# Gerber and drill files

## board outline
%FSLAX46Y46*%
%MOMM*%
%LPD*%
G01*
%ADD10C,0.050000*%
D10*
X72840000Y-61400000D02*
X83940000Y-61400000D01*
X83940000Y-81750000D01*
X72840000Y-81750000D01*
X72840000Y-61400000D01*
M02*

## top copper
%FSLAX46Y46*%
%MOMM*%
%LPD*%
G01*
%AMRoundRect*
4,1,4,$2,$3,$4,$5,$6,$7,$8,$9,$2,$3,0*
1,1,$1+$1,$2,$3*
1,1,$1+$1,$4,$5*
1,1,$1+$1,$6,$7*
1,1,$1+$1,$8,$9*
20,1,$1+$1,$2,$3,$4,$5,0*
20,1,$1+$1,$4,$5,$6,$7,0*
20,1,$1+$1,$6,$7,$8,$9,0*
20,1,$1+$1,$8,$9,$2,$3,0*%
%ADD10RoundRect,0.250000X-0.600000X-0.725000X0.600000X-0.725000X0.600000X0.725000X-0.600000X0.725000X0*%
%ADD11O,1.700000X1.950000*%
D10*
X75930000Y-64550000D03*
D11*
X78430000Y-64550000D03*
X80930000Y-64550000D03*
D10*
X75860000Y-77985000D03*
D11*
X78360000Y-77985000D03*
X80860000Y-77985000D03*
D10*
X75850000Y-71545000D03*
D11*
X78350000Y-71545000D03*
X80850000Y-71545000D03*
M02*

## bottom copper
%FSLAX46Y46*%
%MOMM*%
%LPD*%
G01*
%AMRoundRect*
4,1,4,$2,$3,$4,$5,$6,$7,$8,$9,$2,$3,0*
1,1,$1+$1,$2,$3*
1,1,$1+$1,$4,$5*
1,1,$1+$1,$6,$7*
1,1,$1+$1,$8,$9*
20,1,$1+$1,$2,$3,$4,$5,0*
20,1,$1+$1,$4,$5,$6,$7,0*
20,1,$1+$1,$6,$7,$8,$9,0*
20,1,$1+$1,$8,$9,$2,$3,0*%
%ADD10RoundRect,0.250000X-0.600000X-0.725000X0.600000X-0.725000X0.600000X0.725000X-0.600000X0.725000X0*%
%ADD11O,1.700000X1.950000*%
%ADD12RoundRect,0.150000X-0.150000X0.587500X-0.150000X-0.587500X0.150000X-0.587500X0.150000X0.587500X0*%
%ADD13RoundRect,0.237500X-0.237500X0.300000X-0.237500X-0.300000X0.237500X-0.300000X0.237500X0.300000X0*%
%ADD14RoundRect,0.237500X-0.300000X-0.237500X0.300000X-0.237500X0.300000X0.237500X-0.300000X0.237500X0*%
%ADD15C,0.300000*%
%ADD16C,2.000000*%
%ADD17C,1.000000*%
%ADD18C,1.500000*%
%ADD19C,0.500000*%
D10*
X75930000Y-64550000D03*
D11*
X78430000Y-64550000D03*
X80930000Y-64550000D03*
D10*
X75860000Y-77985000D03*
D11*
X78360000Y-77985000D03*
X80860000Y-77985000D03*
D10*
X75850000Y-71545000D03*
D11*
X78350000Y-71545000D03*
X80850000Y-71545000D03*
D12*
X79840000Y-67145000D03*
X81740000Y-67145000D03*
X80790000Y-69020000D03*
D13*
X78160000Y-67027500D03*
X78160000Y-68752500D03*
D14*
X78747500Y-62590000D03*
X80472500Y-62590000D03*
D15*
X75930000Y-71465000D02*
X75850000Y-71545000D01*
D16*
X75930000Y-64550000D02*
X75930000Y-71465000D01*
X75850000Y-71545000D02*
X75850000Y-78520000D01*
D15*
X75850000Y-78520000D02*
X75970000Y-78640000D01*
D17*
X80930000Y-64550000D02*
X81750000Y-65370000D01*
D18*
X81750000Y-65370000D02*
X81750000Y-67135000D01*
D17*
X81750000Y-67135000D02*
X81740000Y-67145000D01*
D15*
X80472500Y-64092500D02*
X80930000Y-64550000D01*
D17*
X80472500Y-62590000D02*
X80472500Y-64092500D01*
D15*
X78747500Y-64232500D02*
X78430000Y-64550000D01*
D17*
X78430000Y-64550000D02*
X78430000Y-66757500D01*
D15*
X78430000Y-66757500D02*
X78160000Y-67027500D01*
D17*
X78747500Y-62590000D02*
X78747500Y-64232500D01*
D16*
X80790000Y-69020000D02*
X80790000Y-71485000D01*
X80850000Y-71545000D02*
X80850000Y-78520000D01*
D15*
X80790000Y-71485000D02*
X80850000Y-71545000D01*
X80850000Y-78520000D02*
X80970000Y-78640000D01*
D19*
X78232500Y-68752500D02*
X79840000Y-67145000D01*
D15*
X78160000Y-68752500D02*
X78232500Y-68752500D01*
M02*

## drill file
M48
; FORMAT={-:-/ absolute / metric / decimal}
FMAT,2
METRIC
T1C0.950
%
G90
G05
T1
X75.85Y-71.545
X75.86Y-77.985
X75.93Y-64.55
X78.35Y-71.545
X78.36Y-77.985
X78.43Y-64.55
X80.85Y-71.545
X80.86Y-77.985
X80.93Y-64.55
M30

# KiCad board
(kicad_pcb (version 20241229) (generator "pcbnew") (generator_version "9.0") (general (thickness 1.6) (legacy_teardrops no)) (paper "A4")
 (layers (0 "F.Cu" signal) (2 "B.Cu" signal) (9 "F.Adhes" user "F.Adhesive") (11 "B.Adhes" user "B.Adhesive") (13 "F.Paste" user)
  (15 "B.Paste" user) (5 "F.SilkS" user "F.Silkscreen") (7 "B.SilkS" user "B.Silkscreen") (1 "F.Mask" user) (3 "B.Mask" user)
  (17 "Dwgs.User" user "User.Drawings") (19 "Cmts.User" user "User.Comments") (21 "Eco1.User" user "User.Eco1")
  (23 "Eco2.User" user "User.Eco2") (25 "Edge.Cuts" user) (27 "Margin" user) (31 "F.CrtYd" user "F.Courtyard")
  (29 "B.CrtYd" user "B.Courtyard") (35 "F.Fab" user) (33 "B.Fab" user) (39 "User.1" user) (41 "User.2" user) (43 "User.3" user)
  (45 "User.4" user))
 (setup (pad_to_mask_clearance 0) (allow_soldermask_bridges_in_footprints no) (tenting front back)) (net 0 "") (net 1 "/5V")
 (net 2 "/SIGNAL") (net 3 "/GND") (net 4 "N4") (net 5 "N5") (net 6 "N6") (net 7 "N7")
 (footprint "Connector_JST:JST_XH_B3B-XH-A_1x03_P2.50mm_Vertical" (layer "F.Cu") (at 75.93 64.55)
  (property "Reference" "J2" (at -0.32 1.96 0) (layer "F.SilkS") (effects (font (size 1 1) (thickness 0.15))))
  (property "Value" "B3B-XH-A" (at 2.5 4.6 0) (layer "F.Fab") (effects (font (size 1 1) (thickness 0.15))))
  (pad "1" thru_hole roundrect (at 0 0) (size 1.7 1.95) (drill 0.95) (layers "*.Cu" "*.Mask") (remove_unused_layers no)
   (roundrect_rratio 0.147059) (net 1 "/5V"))
  (pad "2" thru_hole oval (at 2.5 0) (size 1.7 1.95) (drill 0.95) (layers "*.Cu" "*.Mask") (remove_unused_layers no) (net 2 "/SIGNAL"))
  (pad "3" thru_hole oval (at 5 0) (size 1.7 1.95) (drill 0.95) (layers "*.Cu" "*.Mask") (remove_unused_layers no) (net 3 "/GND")))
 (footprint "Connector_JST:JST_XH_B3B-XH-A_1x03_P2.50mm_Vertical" (layer "F.Cu") (at 75.86 77.985)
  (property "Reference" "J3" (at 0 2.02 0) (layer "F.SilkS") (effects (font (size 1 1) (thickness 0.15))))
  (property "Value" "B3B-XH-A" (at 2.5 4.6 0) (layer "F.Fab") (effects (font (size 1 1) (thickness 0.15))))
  (pad "1" thru_hole roundrect (at 0 0) (size 1.7 1.95) (drill 0.95) (layers "*.Cu" "*.Mask") (remove_unused_layers no)
   (roundrect_rratio 0.147059) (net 1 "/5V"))
  (pad "2" thru_hole oval (at 2.5 0) (size 1.7 1.95) (drill 0.95) (layers "*.Cu" "*.Mask") (remove_unused_layers no) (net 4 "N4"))
  (pad "3" thru_hole oval (at 5 0) (size 1.7 1.95) (drill 0.95) (layers "*.Cu" "*.Mask") (remove_unused_layers no) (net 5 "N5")))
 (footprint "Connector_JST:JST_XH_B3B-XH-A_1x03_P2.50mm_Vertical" (layer "F.Cu") (at 75.85 71.545)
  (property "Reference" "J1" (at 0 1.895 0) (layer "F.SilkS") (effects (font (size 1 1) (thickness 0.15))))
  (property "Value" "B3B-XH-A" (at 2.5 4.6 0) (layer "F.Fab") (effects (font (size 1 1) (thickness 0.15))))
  (pad "1" thru_hole roundrect (at 0 0) (size 1.7 1.95) (drill 0.95) (layers "*.Cu" "*.Mask") (remove_unused_layers no)
   (roundrect_rratio 0.147059) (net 1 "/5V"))
  (pad "2" thru_hole oval (at 2.5 0) (size 1.7 1.95) (drill 0.95) (layers "*.Cu" "*.Mask") (remove_unused_layers no) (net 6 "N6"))
  (pad "3" thru_hole oval (at 5 0) (size 1.7 1.95) (drill 0.95) (layers "*.Cu" "*.Mask") (remove_unused_layers no) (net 5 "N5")))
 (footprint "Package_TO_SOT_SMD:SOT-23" (layer "B.Cu") (at 80.79 68.0825 -90)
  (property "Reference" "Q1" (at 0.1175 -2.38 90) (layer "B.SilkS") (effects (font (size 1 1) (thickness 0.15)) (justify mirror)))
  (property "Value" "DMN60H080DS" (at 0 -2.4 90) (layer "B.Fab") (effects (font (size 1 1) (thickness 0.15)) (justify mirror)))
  (pad "1" smd roundrect (at -0.9375 0.95 270) (size 1.475 0.6) (layers "B.Cu" "B.Mask" "B.Paste") (roundrect_rratio 0.25) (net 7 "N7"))
  (pad "2" smd roundrect (at -0.9375 -0.95 270) (size 1.475 0.6) (layers "B.Cu" "B.Mask" "B.Paste") (roundrect_rratio 0.25) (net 3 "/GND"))
  (pad "3" smd roundrect (at 0.9375 0 270) (size 1.475 0.6) (layers "B.Cu" "B.Mask" "B.Paste") (roundrect_rratio 0.25) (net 5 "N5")))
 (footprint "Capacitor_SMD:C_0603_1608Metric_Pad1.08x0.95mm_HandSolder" (layer "B.Cu") (at 78.16 67.89 -90)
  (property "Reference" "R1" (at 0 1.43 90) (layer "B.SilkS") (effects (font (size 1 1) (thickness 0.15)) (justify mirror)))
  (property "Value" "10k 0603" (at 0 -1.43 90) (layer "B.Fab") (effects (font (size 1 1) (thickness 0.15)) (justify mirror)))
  (pad "1" smd roundrect (at -0.8625 0 270) (size 1.075 0.95) (layers "B.Cu" "B.Mask" "B.Paste") (roundrect_rratio 0.25) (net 2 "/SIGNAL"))
  (pad "2" smd roundrect (at 0.8625 0 270) (size 1.075 0.95) (layers "B.Cu" "B.Mask" "B.Paste") (roundrect_rratio 0.25) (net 7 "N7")))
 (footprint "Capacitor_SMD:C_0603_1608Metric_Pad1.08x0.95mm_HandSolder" (layer "B.Cu") (at 79.61 62.59)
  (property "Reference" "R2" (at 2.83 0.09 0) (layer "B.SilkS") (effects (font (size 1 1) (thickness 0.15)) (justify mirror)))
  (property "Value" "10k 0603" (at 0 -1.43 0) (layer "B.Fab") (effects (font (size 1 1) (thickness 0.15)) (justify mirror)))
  (pad "1" smd roundrect (at -0.8625 0) (size 1.075 0.95) (layers "B.Cu" "B.Mask" "B.Paste") (roundrect_rratio 0.25) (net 2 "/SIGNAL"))
  (pad "2" smd roundrect (at 0.8625 0) (size 1.075 0.95) (layers "B.Cu" "B.Mask" "B.Paste") (roundrect_rratio 0.25) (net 3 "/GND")))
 (gr_rect (start 72.84 61.4) (end 83.94 81.75) (stroke (width 0.05) (type default)) (fill no) (layer "Edge.Cuts"))
 (segment (start 75.93 71.465) (end 75.85 71.545) (width 0.3) (layer "B.Cu") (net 1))
 (segment (start 75.93 64.55) (end 75.93 71.465) (width 2) (layer "B.Cu") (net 1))
 (segment (start 75.85 71.545) (end 75.85 78.52) (width 2) (layer "B.Cu") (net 1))
 (segment (start 75.85 78.52) (end 75.97 78.64) (width 0.3) (layer "B.Cu") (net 1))
 (segment (start 80.93 64.55) (end 81.75 65.37) (width 1) (layer "B.Cu") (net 3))
 (segment (start 81.75 65.37) (end 81.75 67.135) (width 1.5) (layer "B.Cu") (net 3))
 (segment (start 81.75 67.135) (end 81.74 67.145) (width 1) (layer "B.Cu") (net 3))
 (segment (start 80.4725 64.0925) (end 80.93 64.55) (width 0.3) (layer "B.Cu") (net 3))
 (segment (start 80.4725 62.59) (end 80.4725 64.0925) (width 1) (layer "B.Cu") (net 3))
 (segment (start 78.7475 64.2325) (end 78.43 64.55) (width 0.3) (layer "B.Cu") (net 2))
 (segment (start 78.43 64.55) (end 78.43 66.7575) (width 1) (layer "B.Cu") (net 2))
 (segment (start 78.43 66.7575) (end 78.16 67.0275) (width 0.3) (layer "B.Cu") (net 2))
 (segment (start 78.7475 62.59) (end 78.7475 64.2325) (width 1) (layer "B.Cu") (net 2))
 (segment (start 80.79 69.02) (end 80.79 71.485) (width 2) (layer "B.Cu") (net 5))
 (segment (start 80.85 71.545) (end 80.85 78.52) (width 2) (layer "B.Cu") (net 5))
 (segment (start 80.79 71.485) (end 80.85 71.545) (width 0.3) (layer "B.Cu") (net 5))
 (segment (start 80.85 78.52) (end 80.97 78.64) (width 0.3) (layer "B.Cu") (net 5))
 (segment (start 78.2325 68.7525) (end 79.84 67.145) (width 0.5) (layer "B.Cu") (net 7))
 (segment (start 78.16 68.7525) (end 78.2325 68.7525) (width 0.3) (layer "B.Cu") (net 7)))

